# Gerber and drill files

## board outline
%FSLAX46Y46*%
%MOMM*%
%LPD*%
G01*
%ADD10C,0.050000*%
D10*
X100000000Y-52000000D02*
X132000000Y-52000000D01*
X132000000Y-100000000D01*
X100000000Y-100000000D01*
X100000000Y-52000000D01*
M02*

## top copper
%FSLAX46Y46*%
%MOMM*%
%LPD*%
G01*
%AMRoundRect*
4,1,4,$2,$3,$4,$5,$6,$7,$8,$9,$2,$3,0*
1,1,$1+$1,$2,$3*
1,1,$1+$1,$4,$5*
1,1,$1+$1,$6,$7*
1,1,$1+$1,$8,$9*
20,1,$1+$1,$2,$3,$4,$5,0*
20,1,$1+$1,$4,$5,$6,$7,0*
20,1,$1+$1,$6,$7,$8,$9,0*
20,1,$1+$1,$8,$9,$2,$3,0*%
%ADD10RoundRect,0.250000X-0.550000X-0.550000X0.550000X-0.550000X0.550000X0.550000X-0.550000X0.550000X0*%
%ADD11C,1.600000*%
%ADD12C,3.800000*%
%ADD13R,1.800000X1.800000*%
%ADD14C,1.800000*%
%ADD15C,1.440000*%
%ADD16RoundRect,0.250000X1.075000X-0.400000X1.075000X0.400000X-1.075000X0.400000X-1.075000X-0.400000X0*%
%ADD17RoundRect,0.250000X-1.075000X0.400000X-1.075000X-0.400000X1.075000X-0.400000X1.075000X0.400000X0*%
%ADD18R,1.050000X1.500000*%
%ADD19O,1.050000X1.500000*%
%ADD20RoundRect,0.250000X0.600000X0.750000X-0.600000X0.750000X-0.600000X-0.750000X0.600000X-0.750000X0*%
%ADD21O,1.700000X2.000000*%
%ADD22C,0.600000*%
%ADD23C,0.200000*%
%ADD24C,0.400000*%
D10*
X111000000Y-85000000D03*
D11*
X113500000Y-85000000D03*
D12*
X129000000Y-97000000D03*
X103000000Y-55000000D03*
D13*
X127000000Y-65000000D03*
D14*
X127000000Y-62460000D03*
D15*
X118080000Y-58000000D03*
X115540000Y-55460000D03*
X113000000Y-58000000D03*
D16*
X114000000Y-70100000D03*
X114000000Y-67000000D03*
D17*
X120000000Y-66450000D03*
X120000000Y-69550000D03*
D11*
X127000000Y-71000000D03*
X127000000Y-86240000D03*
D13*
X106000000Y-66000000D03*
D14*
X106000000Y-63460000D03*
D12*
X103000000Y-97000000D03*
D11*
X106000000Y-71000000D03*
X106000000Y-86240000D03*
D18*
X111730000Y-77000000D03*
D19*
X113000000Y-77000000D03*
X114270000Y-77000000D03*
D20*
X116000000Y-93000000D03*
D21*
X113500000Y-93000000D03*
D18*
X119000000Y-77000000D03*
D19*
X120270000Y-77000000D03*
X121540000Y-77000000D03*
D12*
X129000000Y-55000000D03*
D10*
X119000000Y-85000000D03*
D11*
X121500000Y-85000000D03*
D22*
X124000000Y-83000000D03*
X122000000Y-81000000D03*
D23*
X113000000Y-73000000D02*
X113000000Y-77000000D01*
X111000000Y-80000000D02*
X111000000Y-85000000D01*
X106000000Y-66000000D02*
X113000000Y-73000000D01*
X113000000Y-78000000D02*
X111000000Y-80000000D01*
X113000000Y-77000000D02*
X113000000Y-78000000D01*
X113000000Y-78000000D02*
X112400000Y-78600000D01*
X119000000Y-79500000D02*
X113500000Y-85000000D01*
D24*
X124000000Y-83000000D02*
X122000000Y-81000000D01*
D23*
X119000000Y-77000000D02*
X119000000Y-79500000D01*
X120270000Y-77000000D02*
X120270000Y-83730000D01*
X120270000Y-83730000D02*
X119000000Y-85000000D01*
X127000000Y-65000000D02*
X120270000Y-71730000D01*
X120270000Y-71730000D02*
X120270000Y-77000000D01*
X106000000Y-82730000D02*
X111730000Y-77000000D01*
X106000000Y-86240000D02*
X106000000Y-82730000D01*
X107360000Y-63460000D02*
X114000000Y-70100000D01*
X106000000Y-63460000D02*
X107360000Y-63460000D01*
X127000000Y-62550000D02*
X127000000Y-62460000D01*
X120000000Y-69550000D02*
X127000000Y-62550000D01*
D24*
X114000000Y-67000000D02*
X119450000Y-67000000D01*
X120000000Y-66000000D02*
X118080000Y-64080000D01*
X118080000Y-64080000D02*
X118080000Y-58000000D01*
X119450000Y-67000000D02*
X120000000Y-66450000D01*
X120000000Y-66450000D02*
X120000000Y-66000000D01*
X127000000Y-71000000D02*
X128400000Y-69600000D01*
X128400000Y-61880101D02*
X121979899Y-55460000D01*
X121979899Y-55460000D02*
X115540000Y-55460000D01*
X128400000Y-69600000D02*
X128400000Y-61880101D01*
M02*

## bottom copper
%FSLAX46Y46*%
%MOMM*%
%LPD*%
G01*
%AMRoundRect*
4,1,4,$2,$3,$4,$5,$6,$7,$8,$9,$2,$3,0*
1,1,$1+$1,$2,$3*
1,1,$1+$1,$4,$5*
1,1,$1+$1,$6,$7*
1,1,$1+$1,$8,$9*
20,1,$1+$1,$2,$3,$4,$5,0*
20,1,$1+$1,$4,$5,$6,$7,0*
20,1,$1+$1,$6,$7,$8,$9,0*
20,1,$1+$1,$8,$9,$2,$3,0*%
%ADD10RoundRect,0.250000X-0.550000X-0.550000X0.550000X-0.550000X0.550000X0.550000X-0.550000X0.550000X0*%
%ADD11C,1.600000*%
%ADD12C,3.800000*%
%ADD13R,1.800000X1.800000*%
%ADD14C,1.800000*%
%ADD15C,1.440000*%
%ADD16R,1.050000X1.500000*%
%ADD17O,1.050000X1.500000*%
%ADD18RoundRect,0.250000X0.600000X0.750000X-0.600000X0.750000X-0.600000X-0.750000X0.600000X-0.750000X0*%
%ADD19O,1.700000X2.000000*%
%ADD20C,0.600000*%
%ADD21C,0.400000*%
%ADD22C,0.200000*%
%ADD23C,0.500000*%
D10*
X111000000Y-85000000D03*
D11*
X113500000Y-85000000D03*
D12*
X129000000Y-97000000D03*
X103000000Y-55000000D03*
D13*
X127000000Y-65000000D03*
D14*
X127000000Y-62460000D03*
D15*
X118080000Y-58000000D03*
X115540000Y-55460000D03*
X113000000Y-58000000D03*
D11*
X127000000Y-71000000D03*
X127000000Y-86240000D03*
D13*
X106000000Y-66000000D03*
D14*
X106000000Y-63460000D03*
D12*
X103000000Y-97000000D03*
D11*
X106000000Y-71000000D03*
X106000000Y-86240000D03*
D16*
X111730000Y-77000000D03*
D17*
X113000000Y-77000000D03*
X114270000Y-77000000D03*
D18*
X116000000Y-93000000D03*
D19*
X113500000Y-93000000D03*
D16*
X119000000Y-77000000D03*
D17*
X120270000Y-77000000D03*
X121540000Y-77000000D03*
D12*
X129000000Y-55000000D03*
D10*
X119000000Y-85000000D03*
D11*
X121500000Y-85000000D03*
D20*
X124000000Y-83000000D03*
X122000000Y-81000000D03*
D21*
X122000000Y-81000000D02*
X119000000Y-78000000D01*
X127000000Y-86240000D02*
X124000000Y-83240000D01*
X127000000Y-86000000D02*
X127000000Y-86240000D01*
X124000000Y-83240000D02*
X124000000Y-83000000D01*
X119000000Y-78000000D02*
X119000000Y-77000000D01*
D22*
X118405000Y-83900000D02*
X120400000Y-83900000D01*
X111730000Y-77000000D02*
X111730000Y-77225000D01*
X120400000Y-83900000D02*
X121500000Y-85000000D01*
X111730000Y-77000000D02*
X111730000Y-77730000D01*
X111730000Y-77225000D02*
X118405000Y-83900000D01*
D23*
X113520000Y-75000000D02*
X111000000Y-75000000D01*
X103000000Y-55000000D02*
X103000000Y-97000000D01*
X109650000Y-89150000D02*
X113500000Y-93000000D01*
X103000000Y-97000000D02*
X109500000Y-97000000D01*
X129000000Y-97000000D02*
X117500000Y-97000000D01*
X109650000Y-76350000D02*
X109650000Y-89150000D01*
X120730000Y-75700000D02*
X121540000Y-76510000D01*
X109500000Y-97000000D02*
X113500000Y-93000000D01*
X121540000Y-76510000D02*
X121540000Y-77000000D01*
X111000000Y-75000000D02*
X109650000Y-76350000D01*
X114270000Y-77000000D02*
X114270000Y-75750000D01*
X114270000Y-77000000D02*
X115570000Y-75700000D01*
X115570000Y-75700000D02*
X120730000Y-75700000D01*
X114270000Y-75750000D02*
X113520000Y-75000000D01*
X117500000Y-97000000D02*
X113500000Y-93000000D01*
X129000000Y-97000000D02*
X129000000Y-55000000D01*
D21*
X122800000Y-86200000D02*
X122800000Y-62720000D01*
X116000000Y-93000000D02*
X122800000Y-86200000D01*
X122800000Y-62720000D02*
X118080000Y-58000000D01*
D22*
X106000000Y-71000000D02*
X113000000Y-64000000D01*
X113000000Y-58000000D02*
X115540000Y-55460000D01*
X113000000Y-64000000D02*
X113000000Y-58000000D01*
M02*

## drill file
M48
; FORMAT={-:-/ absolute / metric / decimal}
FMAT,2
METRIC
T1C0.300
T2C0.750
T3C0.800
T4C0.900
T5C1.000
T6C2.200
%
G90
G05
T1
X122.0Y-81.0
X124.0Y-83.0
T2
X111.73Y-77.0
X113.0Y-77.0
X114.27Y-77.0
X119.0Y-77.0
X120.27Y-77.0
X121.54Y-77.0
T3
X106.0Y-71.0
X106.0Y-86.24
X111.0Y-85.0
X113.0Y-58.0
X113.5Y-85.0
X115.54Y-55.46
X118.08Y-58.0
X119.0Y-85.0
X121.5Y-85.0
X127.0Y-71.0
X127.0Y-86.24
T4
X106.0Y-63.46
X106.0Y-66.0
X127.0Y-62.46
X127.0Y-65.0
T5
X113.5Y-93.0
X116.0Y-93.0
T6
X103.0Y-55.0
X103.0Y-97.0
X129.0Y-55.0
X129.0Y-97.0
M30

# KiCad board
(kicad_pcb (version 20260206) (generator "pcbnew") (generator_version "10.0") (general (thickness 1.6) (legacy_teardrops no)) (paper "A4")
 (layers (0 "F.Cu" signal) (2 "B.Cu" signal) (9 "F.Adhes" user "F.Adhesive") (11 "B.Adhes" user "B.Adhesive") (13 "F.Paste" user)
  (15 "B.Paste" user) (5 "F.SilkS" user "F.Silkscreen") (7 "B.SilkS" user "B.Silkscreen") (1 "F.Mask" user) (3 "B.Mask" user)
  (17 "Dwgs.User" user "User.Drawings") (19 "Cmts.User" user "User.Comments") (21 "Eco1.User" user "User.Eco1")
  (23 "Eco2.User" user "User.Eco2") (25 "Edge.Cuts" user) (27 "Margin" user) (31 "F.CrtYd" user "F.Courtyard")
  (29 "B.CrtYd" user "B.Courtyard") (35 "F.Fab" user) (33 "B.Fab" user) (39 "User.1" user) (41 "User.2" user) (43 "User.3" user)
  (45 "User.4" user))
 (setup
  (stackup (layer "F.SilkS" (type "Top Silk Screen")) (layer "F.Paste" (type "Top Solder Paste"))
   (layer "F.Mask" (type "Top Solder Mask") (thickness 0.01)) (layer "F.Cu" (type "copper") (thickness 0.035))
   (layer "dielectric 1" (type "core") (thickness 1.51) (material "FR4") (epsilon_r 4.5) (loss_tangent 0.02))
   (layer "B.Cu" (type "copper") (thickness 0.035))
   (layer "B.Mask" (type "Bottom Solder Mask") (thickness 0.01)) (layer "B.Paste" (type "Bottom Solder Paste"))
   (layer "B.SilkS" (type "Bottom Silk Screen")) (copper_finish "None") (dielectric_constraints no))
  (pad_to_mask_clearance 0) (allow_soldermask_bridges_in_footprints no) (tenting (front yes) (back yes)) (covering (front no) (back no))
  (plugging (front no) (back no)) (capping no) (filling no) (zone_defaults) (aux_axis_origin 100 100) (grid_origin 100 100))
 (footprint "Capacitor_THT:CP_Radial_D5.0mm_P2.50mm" (layer "F.Cu") (at 111 85)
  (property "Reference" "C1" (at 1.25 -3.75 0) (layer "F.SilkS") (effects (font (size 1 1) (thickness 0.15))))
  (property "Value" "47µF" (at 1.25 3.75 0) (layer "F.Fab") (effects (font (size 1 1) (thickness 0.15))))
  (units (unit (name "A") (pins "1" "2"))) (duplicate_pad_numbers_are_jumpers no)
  (pad "1" thru_hole roundrect (at 0 0) (size 1.6 1.6) (drill 0.8) (layers "*.Cu" "*.Mask") (remove_unused_layers no)
   (roundrect_rratio 0.15625) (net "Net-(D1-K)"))
  (pad "2" thru_hole circle (at 2.5 0) (size 1.6 1.6) (drill 0.8) (layers "*.Cu" "*.Mask") (remove_unused_layers no) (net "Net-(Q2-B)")))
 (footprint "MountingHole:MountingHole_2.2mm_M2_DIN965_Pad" (layer "F.Cu") (at 129 97)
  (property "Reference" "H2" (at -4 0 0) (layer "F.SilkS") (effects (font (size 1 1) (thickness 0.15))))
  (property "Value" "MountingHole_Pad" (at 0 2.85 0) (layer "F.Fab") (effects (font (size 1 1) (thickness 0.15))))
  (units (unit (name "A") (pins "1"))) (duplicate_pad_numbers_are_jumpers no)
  (pad "1" thru_hole circle (at 0 0) (size 3.8 3.8) (drill 2.2) (layers "*.Cu" "*.Mask") (remove_unused_layers no) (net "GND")
   (zone_connect 2)))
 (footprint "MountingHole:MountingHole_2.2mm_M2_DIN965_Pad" (layer "F.Cu") (at 103 55)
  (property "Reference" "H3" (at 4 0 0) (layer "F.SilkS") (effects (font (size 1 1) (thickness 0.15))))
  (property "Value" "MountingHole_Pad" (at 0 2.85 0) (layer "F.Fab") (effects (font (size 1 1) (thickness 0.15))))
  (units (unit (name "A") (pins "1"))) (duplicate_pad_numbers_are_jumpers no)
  (pad "1" thru_hole circle (at 0 0) (size 3.8 3.8) (drill 2.2) (layers "*.Cu" "*.Mask") (remove_unused_layers no) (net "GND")
   (zone_connect 2)))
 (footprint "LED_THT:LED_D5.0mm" (layer "F.Cu") (at 127 65 90)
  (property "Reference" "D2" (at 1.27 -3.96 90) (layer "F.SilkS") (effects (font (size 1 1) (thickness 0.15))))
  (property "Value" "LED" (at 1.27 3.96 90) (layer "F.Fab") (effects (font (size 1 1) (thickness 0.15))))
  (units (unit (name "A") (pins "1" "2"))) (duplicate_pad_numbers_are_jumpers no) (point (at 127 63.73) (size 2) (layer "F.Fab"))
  (pad "1" thru_hole rect (at 0 0 90) (size 1.8 1.8) (drill 0.9) (layers "*.Cu" "*.Mask") (remove_unused_layers no) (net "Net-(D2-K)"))
  (pad "2" thru_hole circle (at 2.54 0 90) (size 1.8 1.8) (drill 0.9) (layers "*.Cu" "*.Mask") (remove_unused_layers no) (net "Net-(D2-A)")))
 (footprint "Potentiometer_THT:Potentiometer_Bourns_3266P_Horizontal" (layer "F.Cu") (at 118.08 58 -90)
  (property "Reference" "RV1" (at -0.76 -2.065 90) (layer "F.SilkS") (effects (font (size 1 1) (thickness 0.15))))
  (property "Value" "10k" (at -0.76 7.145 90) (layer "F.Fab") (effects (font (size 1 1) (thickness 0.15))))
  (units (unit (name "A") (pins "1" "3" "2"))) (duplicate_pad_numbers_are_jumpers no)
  (pad "1" thru_hole circle (at 0 0 270) (size 1.44 1.44) (drill 0.8) (layers "*.Cu" "*.Mask") (remove_unused_layers no) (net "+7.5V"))
  (pad "2" thru_hole circle (at -2.54 2.54 270) (size 1.44 1.44) (drill 0.8) (layers "*.Cu" "*.Mask") (remove_unused_layers no)
   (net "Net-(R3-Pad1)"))
  (pad "3" thru_hole circle (at 0 5.08 270) (size 1.44 1.44) (drill 0.8) (layers "*.Cu" "*.Mask") (remove_unused_layers no)
   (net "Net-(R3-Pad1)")))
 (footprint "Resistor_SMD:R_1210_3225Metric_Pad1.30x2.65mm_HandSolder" (layer "F.Cu") (at 114 68.55 90)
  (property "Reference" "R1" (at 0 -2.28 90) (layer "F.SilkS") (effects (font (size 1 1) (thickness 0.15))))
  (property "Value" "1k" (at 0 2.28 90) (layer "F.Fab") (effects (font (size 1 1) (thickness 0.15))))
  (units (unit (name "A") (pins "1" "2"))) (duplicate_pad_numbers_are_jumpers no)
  (pad "1" smd roundrect (at -1.55 0 90) (size 1.3 2.65) (layers "F.Cu" "F.Mask" "F.Paste") (roundrect_rratio 0.192308) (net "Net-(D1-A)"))
  (pad "2" smd roundrect (at 1.55 0 90) (size 1.3 2.65) (layers "F.Cu" "F.Mask" "F.Paste") (roundrect_rratio 0.192308) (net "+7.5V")))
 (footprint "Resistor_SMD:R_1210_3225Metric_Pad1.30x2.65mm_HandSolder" (layer "F.Cu") (at 120 68 -90)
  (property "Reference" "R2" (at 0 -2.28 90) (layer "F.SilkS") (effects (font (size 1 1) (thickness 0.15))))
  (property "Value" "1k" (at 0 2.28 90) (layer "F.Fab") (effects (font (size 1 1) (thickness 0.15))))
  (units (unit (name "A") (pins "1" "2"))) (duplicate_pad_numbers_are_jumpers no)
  (pad "1" smd roundrect (at -1.55 0 270) (size 1.3 2.65) (layers "F.Cu" "F.Mask" "F.Paste") (roundrect_rratio 0.192308) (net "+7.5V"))
  (pad "2" smd roundrect (at 1.55 0 270) (size 1.3 2.65) (layers "F.Cu" "F.Mask" "F.Paste") (roundrect_rratio 0.192308) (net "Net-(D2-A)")))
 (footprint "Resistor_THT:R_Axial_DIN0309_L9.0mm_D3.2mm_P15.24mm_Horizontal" (layer "F.Cu") (at 127 71 -90)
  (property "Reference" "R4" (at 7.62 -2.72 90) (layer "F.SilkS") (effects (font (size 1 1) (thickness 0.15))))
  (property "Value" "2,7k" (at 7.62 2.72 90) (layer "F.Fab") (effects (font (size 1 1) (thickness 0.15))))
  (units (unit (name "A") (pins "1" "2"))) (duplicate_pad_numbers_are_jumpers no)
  (pad "1" thru_hole circle (at 0 0 270) (size 1.6 1.6) (drill 0.8) (layers "*.Cu" "*.Mask") (remove_unused_layers no) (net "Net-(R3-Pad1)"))
  (pad "2" thru_hole circle (at 15.24 0 270) (size 1.6 1.6) (drill 0.8) (layers "*.Cu" "*.Mask") (remove_unused_layers no)
   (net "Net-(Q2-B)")))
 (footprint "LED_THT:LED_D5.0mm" (layer "F.Cu") (at 106 66 90)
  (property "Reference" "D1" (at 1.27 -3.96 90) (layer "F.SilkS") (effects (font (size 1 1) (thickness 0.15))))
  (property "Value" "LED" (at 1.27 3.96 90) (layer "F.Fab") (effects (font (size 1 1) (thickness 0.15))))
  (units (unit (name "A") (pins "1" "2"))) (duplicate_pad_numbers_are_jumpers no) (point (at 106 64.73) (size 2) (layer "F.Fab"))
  (pad "1" thru_hole rect (at 0 0 90) (size 1.8 1.8) (drill 0.9) (layers "*.Cu" "*.Mask") (remove_unused_layers no) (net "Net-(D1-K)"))
  (pad "2" thru_hole circle (at 2.54 0 90) (size 1.8 1.8) (drill 0.9) (layers "*.Cu" "*.Mask") (remove_unused_layers no) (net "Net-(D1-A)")))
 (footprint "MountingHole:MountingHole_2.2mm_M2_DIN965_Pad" (layer "F.Cu") (at 103 97)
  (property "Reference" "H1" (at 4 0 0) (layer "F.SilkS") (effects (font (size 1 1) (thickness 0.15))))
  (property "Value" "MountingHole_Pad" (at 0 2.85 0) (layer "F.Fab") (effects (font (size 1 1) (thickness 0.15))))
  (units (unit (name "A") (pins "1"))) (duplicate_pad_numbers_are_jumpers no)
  (pad "1" thru_hole circle (at 0 0) (size 3.8 3.8) (drill 2.2) (layers "*.Cu" "*.Mask") (remove_unused_layers no) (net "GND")
   (zone_connect 2)))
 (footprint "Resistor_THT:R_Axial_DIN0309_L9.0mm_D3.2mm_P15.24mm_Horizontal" (layer "F.Cu") (at 106 71 -90)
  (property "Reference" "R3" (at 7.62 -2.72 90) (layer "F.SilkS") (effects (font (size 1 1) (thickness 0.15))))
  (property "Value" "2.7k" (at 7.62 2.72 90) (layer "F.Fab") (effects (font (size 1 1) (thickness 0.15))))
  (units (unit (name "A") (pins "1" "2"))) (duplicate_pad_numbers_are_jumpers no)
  (pad "1" thru_hole circle (at 0 0 270) (size 1.6 1.6) (drill 0.8) (layers "*.Cu" "*.Mask") (remove_unused_layers no) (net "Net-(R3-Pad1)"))
  (pad "2" thru_hole circle (at 15.24 0 270) (size 1.6 1.6) (drill 0.8) (layers "*.Cu" "*.Mask") (remove_unused_layers no)
   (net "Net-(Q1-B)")))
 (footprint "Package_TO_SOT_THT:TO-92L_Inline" (layer "F.Cu") (at 111.73 77)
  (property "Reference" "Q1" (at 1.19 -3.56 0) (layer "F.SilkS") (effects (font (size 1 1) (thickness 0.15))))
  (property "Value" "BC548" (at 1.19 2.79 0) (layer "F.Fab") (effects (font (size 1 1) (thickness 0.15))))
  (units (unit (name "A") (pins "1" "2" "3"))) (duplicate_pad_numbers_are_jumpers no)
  (pad "1" thru_hole rect (at 0 0) (size 1.05 1.5) (drill 0.75) (layers "*.Cu" "*.Mask") (remove_unused_layers no) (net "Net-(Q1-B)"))
  (pad "2" thru_hole oval (at 1.27 0) (size 1.05 1.5) (drill 0.75) (layers "*.Cu" "*.Mask") (remove_unused_layers no) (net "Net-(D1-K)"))
  (pad "3" thru_hole oval (at 2.54 0) (size 1.05 1.5) (drill 0.75) (layers "*.Cu" "*.Mask") (remove_unused_layers no) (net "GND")))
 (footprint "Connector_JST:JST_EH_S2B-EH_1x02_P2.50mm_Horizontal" (layer "F.Cu") (at 116 93 180)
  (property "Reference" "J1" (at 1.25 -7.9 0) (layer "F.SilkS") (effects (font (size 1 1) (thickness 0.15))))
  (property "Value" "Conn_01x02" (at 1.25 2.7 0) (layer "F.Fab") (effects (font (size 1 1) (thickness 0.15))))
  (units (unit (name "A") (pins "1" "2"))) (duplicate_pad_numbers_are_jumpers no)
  (pad "1" thru_hole roundrect (at 0 0 180) (size 1.7 2) (drill 1) (layers "*.Cu" "*.Mask") (remove_unused_layers no)
   (roundrect_rratio 0.147059) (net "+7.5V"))
  (pad "2" thru_hole oval (at 2.5 0 180) (size 1.7 2) (drill 1) (layers "*.Cu" "*.Mask") (remove_unused_layers no) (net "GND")))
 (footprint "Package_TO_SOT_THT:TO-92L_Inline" (layer "F.Cu") (at 119 77)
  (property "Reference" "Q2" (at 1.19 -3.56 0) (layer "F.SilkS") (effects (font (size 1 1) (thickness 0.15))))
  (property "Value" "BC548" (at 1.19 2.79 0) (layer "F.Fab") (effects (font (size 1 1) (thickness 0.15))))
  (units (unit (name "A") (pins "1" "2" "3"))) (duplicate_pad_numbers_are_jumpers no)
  (pad "1" thru_hole rect (at 0 0) (size 1.05 1.5) (drill 0.75) (layers "*.Cu" "*.Mask") (remove_unused_layers no) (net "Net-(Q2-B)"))
  (pad "2" thru_hole oval (at 1.27 0) (size 1.05 1.5) (drill 0.75) (layers "*.Cu" "*.Mask") (remove_unused_layers no) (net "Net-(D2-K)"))
  (pad "3" thru_hole oval (at 2.54 0) (size 1.05 1.5) (drill 0.75) (layers "*.Cu" "*.Mask") (remove_unused_layers no) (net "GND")))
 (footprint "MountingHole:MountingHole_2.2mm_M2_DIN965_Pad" (layer "F.Cu") (at 129 55)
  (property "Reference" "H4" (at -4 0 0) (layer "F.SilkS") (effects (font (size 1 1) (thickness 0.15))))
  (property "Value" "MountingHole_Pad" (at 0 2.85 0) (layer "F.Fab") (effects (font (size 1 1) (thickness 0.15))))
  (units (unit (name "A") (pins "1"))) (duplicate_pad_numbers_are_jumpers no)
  (pad "1" thru_hole circle (at 0 0) (size 3.8 3.8) (drill 2.2) (layers "*.Cu" "*.Mask") (remove_unused_layers no) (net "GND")
   (zone_connect 2)))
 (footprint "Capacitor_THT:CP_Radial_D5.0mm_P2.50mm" (layer "F.Cu") (at 119 85)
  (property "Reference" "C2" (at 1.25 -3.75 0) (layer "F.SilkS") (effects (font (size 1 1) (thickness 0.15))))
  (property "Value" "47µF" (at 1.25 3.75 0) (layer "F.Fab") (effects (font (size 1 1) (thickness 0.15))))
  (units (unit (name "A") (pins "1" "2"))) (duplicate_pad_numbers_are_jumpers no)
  (pad "1" thru_hole roundrect (at 0 0) (size 1.6 1.6) (drill 0.8) (layers "*.Cu" "*.Mask") (remove_unused_layers no)
   (roundrect_rratio 0.15625) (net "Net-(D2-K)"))
  (pad "2" thru_hole circle (at 2.5 0) (size 1.6 1.6) (drill 0.8) (layers "*.Cu" "*.Mask") (remove_unused_layers no) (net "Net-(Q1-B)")))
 (gr_rect (start 100 100) (end 132 52) (stroke (width 0.05) (type solid)) (fill no) (layer "Edge.Cuts"))
 (segment (start 113 73) (end 113 77) (width 0.2) (layer "F.Cu") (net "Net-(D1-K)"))
 (segment (start 111 80) (end 111 85) (width 0.2) (layer "F.Cu") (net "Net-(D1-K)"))
 (segment (start 106 66) (end 113 73) (width 0.2) (layer "F.Cu") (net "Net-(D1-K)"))
 (segment (start 113 78) (end 111 80) (width 0.2) (layer "F.Cu") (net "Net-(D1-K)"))
 (segment (start 113 77) (end 113 78) (width 0.2) (layer "F.Cu") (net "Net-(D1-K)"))
 (segment (start 113 78) (end 112.4 78.6) (width 0.2) (layer "F.Cu") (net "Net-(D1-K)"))
 (segment (start 119 79.5) (end 113.5 85) (width 0.2) (layer "F.Cu") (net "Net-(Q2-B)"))
 (segment (start 124 83) (end 122 81) (width 0.4) (layer "F.Cu") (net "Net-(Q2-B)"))
 (segment (start 119 77) (end 119 79.5) (width 0.2) (layer "F.Cu") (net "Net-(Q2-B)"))
 (via (at 124 83) (size 0.6) (drill 0.3) (layers "F.Cu" "B.Cu") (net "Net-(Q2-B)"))
 (via (at 122 81) (size 0.6) (drill 0.3) (layers "F.Cu" "B.Cu") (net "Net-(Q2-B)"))
 (segment (start 122 81) (end 119 78) (width 0.4) (layer "B.Cu") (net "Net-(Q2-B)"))
 (segment (start 127 86.24) (end 124 83.24) (width 0.4) (layer "B.Cu") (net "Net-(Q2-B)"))
 (segment (start 127 86) (end 127 86.24) (width 0.4) (layer "B.Cu") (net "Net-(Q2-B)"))
 (segment (start 124 83.24) (end 124 83) (width 0.4) (layer "B.Cu") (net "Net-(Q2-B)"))
 (segment (start 119 78) (end 119 77) (width 0.4) (layer "B.Cu") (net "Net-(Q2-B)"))
 (segment (start 120.27 77) (end 120.27 83.73) (width 0.2) (layer "F.Cu") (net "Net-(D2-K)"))
 (segment (start 120.27 83.73) (end 119 85) (width 0.2) (layer "F.Cu") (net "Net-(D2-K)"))
 (segment (start 127 65) (end 120.27 71.73) (width 0.2) (layer "F.Cu") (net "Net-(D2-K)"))
 (segment (start 120.27 71.73) (end 120.27 77) (width 0.2) (layer "F.Cu") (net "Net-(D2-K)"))
 (segment (start 106 82.73) (end 111.73 77) (width 0.2) (layer "F.Cu") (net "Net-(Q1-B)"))
 (segment (start 106 86.24) (end 106 82.73) (width 0.2) (layer "F.Cu") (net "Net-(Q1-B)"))
 (segment (start 118.405 83.9) (end 120.4 83.9) (width 0.2) (layer "B.Cu") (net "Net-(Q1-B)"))
 (segment (start 111.73 77) (end 111.73 77.225) (width 0.2) (layer "B.Cu") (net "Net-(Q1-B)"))
 (segment (start 120.4 83.9) (end 121.5 85) (width 0.2) (layer "B.Cu") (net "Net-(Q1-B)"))
 (segment (start 111.73 77) (end 111.73 77.73) (width 0.2) (layer "B.Cu") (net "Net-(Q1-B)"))
 (segment (start 111.73 77.225) (end 118.405 83.9) (width 0.2) (layer "B.Cu") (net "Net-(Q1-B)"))
 (segment (start 107.36 63.46) (end 114 70.1) (width 0.2) (layer "F.Cu") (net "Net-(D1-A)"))
 (segment (start 106 63.46) (end 107.36 63.46) (width 0.2) (layer "F.Cu") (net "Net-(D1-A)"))
 (segment (start 127 62.55) (end 127 62.46) (width 0.2) (layer "F.Cu") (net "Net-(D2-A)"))
 (segment (start 120 69.55) (end 127 62.55) (width 0.2) (layer "F.Cu") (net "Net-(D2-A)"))
 (segment (start 113.52 75) (end 111 75) (width 0.5) (layer "B.Cu") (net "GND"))
 (segment (start 103 55) (end 103 97) (width 0.5) (layer "B.Cu") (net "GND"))
 (segment (start 109.65 89.15) (end 113.5 93) (width 0.5) (layer "B.Cu") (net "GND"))
 (segment (start 103 97) (end 109.5 97) (width 0.5) (layer "B.Cu") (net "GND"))
 (segment (start 129 97) (end 117.5 97) (width 0.5) (layer "B.Cu") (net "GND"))
 (segment (start 109.65 76.35) (end 109.65 89.15) (width 0.5) (layer "B.Cu") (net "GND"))
 (segment (start 120.73 75.7) (end 121.54 76.51) (width 0.5) (layer "B.Cu") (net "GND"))
 (segment (start 109.5 97) (end 113.5 93) (width 0.5) (layer "B.Cu") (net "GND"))
 (segment (start 121.54 76.51) (end 121.54 77) (width 0.5) (layer "B.Cu") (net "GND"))
 (segment (start 111 75) (end 109.65 76.35) (width 0.5) (layer "B.Cu") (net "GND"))
 (segment (start 114.27 77) (end 114.27 75.75) (width 0.5) (layer "B.Cu") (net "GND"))
 (segment (start 114.27 77) (end 115.57 75.7) (width 0.5) (layer "B.Cu") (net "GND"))
 (segment (start 115.57 75.7) (end 120.73 75.7) (width 0.5) (layer "B.Cu") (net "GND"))
 (segment (start 114.27 75.75) (end 113.52 75) (width 0.5) (layer "B.Cu") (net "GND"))
 (segment (start 117.5 97) (end 113.5 93) (width 0.5) (layer "B.Cu") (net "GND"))
 (segment (start 129 97) (end 129 55) (width 0.5) (layer "B.Cu") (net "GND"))
 (segment (start 114 67) (end 119.45 67) (width 0.4) (layer "F.Cu") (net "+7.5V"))
 (segment (start 120 66) (end 118.08 64.08) (width 0.4) (layer "F.Cu") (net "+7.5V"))
 (segment (start 118.08 64.08) (end 118.08 58) (width 0.4) (layer "F.Cu") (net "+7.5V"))
 (segment (start 119.45 67) (end 120 66.45) (width 0.4) (layer "F.Cu") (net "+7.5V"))
 (segment (start 120 66.45) (end 120 66) (width 0.4) (layer "F.Cu") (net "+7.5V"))
 (segment (start 122.8 86.2) (end 122.8 62.72) (width 0.4) (layer "B.Cu") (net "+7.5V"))
 (segment (start 116 93) (end 122.8 86.2) (width 0.4) (layer "B.Cu") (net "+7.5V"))
 (segment (start 122.8 62.72) (end 118.08 58) (width 0.4) (layer "B.Cu") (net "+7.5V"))
 (segment (start 127 71) (end 128.4 69.6) (width 0.4) (layer "F.Cu") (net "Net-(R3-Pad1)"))
 (segment (start 128.4 61.880101) (end 121.979899 55.46) (width 0.4) (layer "F.Cu") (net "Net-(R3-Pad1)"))
 (segment (start 121.979899 55.46) (end 115.54 55.46) (width 0.4) (layer "F.Cu") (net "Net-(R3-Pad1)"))
 (segment (start 128.4 69.6) (end 128.4 61.880101) (width 0.4) (layer "F.Cu") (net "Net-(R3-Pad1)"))
 (segment (start 106 71) (end 113 64) (width 0.2) (layer "B.Cu") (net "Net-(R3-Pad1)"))
 (segment (start 113 58) (end 115.54 55.46) (width 0.2) (layer "B.Cu") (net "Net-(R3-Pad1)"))
 (segment (start 113 64) (end 113 58) (width 0.2) (layer "B.Cu") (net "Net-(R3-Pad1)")))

